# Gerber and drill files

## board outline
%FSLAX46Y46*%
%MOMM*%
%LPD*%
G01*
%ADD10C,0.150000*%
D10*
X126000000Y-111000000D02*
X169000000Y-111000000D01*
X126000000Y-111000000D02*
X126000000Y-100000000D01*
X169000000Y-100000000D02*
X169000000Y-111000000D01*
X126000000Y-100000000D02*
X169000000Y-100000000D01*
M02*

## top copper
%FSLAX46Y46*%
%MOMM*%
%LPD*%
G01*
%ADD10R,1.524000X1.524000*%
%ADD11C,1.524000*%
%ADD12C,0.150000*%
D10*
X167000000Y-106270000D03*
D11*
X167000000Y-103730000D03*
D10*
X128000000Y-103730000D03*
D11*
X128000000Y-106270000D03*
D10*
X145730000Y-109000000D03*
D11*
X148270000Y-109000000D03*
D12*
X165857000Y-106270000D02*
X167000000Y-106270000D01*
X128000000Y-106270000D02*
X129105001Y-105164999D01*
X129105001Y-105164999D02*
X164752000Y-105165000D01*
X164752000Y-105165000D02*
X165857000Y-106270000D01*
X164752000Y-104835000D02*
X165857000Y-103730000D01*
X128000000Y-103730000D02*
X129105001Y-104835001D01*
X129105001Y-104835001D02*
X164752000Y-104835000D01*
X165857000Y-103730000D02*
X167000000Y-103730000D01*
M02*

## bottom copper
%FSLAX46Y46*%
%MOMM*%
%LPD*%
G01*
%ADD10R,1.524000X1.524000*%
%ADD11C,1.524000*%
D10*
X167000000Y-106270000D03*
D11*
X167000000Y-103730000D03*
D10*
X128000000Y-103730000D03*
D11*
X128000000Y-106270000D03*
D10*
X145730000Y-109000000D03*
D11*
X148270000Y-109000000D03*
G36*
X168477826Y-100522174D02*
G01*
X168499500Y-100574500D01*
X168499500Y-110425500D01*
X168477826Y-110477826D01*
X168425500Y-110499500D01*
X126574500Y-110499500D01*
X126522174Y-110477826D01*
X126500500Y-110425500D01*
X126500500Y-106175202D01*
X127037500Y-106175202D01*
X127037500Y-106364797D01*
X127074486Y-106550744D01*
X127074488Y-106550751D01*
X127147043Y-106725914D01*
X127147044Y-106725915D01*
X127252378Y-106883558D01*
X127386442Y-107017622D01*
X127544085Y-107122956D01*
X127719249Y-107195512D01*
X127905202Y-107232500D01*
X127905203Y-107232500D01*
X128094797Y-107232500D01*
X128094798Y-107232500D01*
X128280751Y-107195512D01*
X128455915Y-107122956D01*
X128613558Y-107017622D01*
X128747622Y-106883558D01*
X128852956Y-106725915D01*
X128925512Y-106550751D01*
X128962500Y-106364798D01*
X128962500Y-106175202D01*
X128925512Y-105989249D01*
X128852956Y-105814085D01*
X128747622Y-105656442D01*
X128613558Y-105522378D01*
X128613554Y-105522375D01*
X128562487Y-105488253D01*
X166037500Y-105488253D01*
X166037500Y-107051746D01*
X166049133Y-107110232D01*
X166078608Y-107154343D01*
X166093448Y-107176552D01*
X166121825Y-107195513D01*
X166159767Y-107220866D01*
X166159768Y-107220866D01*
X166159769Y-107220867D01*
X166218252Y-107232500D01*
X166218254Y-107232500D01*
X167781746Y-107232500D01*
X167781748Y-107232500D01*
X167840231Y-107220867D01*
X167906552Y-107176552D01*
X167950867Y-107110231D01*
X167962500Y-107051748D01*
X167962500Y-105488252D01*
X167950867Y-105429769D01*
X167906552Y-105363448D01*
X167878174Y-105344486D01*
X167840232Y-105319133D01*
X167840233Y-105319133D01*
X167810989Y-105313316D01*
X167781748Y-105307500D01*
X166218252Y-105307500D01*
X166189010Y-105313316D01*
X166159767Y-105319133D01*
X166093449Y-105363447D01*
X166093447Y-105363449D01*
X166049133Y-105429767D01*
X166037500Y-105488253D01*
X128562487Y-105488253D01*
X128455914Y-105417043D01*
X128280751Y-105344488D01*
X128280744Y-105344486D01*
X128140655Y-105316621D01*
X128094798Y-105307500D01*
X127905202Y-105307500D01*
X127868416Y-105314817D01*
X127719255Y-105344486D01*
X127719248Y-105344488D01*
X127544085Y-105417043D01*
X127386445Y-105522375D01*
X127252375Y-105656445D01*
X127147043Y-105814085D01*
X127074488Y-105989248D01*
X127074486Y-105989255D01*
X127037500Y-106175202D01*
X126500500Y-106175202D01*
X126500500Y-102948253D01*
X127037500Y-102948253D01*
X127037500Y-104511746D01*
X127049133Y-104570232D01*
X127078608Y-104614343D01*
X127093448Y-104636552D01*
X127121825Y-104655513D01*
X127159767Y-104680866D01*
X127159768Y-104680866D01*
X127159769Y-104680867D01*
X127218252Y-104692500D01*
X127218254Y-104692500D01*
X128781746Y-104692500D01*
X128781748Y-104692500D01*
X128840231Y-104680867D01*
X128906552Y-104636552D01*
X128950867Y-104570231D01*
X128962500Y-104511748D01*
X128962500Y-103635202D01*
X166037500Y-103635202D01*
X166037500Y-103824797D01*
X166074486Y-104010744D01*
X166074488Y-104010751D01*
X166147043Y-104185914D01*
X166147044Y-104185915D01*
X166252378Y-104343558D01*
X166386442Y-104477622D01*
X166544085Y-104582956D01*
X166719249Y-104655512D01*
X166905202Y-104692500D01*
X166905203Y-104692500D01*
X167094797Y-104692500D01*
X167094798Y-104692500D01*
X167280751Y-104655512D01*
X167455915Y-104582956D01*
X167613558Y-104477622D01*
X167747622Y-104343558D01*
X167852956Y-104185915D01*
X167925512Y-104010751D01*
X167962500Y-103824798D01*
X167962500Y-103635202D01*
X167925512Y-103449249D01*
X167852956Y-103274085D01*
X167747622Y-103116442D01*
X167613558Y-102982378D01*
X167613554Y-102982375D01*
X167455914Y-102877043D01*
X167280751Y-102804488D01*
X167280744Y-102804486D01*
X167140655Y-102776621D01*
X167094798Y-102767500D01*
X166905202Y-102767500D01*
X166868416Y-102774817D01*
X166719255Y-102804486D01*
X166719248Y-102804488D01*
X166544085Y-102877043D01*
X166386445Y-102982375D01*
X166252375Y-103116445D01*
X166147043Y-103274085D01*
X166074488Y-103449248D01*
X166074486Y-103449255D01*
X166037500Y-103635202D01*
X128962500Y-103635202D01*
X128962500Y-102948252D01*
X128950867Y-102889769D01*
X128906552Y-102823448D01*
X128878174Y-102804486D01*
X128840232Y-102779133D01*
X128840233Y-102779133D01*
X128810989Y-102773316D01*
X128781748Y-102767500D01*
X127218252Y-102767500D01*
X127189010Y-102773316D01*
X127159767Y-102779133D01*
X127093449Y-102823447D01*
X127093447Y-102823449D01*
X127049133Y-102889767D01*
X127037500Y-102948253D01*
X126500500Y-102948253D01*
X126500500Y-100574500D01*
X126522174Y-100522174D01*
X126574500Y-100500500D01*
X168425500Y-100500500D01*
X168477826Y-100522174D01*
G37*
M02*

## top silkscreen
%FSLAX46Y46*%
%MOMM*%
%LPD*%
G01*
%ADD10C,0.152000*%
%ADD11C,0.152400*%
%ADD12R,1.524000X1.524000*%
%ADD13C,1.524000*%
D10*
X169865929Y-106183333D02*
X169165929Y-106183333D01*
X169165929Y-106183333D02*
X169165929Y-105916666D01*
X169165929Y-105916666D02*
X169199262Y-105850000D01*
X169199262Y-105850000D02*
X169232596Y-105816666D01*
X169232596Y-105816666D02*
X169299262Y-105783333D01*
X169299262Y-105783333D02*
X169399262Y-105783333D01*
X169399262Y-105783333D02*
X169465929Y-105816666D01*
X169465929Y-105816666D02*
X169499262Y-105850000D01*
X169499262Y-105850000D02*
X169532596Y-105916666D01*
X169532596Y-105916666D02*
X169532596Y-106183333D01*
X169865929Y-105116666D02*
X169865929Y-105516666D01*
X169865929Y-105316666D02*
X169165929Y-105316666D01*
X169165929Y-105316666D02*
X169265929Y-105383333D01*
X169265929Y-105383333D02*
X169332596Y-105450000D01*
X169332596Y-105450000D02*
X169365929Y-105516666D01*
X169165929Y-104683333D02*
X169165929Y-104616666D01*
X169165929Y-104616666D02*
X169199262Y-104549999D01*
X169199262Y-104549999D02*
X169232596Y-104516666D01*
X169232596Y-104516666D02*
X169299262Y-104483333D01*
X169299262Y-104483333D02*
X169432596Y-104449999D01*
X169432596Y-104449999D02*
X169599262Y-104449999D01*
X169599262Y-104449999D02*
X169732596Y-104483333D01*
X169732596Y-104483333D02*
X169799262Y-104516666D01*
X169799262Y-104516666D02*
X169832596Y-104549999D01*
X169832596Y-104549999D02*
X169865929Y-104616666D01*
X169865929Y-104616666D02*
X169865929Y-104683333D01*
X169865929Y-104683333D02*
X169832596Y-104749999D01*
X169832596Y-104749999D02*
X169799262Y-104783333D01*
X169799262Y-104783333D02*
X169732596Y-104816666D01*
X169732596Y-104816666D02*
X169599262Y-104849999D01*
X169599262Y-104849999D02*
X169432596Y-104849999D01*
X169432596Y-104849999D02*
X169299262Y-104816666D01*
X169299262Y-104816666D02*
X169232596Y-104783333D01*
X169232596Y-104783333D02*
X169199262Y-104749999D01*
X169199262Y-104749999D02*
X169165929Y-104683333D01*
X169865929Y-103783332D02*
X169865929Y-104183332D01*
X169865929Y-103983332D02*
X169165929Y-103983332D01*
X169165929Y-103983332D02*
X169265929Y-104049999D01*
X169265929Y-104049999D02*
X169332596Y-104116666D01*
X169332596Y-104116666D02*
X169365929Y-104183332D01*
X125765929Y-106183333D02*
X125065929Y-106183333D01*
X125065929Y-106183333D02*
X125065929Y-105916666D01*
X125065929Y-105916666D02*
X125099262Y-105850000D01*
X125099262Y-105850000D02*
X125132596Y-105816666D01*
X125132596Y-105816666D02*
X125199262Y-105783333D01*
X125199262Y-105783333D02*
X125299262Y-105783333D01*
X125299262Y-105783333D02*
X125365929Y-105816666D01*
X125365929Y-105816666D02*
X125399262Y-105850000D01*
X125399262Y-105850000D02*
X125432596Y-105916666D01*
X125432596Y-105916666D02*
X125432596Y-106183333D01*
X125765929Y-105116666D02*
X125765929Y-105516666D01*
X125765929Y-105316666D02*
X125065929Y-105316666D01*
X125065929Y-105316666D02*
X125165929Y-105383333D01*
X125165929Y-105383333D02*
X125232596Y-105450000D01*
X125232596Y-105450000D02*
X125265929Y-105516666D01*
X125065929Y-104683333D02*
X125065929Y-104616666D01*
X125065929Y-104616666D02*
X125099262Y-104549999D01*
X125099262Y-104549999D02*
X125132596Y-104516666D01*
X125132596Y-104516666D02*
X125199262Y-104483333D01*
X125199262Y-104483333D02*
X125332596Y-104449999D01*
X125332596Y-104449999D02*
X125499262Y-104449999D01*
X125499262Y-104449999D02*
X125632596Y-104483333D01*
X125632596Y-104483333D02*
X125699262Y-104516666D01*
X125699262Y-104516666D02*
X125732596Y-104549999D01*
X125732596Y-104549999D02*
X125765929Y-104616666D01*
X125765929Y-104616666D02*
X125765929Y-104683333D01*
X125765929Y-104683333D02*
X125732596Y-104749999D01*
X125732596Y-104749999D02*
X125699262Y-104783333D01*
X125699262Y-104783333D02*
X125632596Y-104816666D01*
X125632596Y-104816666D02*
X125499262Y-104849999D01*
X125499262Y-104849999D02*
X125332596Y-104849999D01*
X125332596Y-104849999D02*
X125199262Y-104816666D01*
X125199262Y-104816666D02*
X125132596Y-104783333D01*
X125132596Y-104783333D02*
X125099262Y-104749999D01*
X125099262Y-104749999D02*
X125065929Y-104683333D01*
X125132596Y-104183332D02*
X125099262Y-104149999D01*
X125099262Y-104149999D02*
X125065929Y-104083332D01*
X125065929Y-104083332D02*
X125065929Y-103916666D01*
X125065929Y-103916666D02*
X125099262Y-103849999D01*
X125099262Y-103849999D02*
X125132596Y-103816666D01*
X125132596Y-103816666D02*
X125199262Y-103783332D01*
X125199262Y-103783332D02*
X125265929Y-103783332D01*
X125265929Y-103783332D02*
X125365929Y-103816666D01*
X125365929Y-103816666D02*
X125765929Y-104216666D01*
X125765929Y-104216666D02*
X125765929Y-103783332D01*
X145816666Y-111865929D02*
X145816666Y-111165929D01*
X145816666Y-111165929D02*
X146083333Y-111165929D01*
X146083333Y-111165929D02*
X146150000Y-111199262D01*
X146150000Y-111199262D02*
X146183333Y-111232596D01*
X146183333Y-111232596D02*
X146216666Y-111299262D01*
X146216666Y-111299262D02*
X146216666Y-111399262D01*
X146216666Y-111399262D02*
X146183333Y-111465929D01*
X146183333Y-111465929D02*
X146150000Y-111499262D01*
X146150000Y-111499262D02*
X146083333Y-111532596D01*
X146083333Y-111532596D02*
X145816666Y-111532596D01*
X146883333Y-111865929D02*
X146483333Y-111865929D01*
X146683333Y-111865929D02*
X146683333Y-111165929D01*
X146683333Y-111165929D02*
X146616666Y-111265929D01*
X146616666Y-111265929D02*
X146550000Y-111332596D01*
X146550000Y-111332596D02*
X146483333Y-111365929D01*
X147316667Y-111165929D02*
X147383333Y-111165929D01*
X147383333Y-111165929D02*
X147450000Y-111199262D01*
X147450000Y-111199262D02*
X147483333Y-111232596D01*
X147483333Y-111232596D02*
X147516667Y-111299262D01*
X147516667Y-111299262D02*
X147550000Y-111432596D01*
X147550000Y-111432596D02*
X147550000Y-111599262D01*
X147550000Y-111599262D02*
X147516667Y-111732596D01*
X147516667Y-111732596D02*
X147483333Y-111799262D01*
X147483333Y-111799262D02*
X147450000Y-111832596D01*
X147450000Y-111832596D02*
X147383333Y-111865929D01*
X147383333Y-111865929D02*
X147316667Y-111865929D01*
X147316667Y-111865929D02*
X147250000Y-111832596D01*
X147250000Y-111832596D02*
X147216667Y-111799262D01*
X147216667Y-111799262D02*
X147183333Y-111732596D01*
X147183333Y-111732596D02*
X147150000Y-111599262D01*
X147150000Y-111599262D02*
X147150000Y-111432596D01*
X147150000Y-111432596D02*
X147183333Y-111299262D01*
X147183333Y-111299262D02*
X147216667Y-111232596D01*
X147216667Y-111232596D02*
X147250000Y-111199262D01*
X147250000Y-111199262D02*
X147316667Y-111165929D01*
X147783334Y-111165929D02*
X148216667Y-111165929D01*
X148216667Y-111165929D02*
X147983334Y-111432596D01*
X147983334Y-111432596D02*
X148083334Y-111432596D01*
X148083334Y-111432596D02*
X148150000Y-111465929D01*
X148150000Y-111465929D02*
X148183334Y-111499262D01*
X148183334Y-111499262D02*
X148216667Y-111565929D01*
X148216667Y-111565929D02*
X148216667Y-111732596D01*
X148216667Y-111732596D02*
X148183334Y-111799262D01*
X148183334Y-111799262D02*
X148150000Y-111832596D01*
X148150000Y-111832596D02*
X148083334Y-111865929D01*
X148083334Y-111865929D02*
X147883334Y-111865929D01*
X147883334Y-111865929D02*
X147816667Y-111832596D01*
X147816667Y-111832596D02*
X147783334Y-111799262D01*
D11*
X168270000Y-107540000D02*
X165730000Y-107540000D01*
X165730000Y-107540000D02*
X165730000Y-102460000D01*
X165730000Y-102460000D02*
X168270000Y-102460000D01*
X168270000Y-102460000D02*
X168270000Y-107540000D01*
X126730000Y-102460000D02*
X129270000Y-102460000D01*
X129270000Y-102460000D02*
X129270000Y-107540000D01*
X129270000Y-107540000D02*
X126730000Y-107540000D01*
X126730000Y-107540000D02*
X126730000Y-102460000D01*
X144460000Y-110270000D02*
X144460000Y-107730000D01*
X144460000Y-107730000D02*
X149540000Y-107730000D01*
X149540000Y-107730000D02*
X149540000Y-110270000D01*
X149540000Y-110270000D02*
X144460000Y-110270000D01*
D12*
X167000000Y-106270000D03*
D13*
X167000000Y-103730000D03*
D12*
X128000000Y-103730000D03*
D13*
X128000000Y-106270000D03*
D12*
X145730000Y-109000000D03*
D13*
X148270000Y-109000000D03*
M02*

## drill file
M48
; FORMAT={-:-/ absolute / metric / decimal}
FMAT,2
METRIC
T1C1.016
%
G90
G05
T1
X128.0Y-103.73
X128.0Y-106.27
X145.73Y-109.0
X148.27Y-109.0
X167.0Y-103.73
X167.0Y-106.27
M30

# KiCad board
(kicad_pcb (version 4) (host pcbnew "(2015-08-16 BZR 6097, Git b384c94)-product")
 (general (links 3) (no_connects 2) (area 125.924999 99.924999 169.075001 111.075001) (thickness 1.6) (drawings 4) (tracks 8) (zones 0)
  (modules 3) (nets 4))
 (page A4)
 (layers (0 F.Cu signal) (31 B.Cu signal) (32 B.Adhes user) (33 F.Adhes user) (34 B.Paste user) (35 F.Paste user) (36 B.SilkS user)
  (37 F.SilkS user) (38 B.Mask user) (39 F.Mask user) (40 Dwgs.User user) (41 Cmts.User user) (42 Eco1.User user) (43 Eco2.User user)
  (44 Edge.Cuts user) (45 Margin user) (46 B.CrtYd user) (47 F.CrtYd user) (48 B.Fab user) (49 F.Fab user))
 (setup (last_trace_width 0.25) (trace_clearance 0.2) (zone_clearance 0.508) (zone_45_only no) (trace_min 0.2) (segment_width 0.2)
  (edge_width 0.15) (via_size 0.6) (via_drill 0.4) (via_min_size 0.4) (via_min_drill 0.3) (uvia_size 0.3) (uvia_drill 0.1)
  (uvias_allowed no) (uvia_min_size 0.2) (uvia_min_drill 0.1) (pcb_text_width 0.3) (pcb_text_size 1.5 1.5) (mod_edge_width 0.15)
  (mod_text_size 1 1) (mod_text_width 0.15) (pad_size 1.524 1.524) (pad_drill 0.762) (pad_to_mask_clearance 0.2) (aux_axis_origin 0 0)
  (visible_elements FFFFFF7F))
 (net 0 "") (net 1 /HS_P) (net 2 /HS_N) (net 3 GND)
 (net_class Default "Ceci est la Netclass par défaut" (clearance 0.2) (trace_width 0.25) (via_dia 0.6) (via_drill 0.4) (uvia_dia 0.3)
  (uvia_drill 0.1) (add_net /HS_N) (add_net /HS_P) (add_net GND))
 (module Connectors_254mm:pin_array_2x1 (layer F.Cu) (at 167 105 90)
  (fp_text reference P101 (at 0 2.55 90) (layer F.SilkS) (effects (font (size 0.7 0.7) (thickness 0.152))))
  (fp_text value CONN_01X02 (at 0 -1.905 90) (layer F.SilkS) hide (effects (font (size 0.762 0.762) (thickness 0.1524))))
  (fp_line (start -2.54 1.27) (end -2.54 -1.27) (layer F.SilkS) (width 0.1524))
  (fp_line (start -2.54 -1.27) (end 2.54 -1.27) (layer F.SilkS) (width 0.1524))
  (fp_line (start 2.54 -1.27) (end 2.54 1.27) (layer F.SilkS) (width 0.1524))
  (fp_line (start 2.54 1.27) (end -2.54 1.27) (layer F.SilkS) (width 0.1524))
  (pad 1 thru_hole rect (at -1.27 0 90) (size 1.524 1.524) (drill 1.016) (layers *.Cu *.Mask F.SilkS) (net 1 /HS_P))
  (pad 2 thru_hole circle (at 1.27 0 90) (size 1.524 1.524) (drill 1.016) (layers *.Cu *.Mask F.SilkS) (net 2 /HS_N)))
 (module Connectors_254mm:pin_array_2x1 (layer F.Cu) (at 128 105 270)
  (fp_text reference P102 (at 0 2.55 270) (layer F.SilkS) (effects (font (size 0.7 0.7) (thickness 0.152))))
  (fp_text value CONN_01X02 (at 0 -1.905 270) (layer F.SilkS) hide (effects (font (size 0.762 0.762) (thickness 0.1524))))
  (fp_line (start -2.54 1.27) (end -2.54 -1.27) (layer F.SilkS) (width 0.1524))
  (fp_line (start -2.54 -1.27) (end 2.54 -1.27) (layer F.SilkS) (width 0.1524))
  (fp_line (start 2.54 -1.27) (end 2.54 1.27) (layer F.SilkS) (width 0.1524))
  (fp_line (start 2.54 1.27) (end -2.54 1.27) (layer F.SilkS) (width 0.1524))
  (pad 1 thru_hole rect (at -1.27 0 270) (size 1.524 1.524) (drill 1.016) (layers *.Cu *.Mask F.SilkS) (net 2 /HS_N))
  (pad 2 thru_hole circle (at 1.27 0 270) (size 1.524 1.524) (drill 1.016) (layers *.Cu *.Mask F.SilkS) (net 1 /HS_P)))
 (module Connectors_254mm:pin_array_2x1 (layer F.Cu) (at 147 109)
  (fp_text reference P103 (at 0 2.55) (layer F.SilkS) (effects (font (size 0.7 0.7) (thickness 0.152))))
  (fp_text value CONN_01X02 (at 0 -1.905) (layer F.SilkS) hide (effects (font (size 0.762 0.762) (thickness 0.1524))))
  (fp_line (start -2.54 1.27) (end -2.54 -1.27) (layer F.SilkS) (width 0.1524))
  (fp_line (start -2.54 -1.27) (end 2.54 -1.27) (layer F.SilkS) (width 0.1524))
  (fp_line (start 2.54 -1.27) (end 2.54 1.27) (layer F.SilkS) (width 0.1524))
  (fp_line (start 2.54 1.27) (end -2.54 1.27) (layer F.SilkS) (width 0.1524))
  (pad 1 thru_hole rect (at -1.27 0) (size 1.524 1.524) (drill 1.016) (layers *.Cu *.Mask F.SilkS) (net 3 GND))
  (pad 2 thru_hole circle (at 1.27 0) (size 1.524 1.524) (drill 1.016) (layers *.Cu *.Mask F.SilkS) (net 3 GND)))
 (gr_line (start 126 111) (end 169 111) (layer Edge.Cuts) (width 0.15))
 (gr_line (start 126 111) (end 126 100) (layer Edge.Cuts) (width 0.15))
 (gr_line (start 169 100) (end 169 111) (layer Edge.Cuts) (width 0.15))
 (gr_line (start 126 100) (end 169 100) (layer Edge.Cuts) (width 0.15))
 (segment (start 165.857 106.27) (end 167 106.27) (width 0.15) (layer F.Cu) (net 1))
 (segment (start 128 106.27) (end 129.105001 105.164999) (width 0.15) (layer F.Cu) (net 1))
 (segment (start 129.105001 105.164999) (end 164.752 105.165) (width 0.15) (layer F.Cu) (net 1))
 (segment (start 164.752 105.165) (end 165.857 106.27) (width 0.15) (layer F.Cu) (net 1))
 (segment (start 164.752 104.835) (end 165.857 103.73) (width 0.15) (layer F.Cu) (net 2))
 (segment (start 128 103.73) (end 129.105001 104.835001) (width 0.15) (layer F.Cu) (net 2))
 (segment (start 129.105001 104.835001) (end 164.752 104.835) (width 0.15) (layer F.Cu) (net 2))
 (segment (start 165.857 103.73) (end 167 103.73) (width 0.15) (layer F.Cu) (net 2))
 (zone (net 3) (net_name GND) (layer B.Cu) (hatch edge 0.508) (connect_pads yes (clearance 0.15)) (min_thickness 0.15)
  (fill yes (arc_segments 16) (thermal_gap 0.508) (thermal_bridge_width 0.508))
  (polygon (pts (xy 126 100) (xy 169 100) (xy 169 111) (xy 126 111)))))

